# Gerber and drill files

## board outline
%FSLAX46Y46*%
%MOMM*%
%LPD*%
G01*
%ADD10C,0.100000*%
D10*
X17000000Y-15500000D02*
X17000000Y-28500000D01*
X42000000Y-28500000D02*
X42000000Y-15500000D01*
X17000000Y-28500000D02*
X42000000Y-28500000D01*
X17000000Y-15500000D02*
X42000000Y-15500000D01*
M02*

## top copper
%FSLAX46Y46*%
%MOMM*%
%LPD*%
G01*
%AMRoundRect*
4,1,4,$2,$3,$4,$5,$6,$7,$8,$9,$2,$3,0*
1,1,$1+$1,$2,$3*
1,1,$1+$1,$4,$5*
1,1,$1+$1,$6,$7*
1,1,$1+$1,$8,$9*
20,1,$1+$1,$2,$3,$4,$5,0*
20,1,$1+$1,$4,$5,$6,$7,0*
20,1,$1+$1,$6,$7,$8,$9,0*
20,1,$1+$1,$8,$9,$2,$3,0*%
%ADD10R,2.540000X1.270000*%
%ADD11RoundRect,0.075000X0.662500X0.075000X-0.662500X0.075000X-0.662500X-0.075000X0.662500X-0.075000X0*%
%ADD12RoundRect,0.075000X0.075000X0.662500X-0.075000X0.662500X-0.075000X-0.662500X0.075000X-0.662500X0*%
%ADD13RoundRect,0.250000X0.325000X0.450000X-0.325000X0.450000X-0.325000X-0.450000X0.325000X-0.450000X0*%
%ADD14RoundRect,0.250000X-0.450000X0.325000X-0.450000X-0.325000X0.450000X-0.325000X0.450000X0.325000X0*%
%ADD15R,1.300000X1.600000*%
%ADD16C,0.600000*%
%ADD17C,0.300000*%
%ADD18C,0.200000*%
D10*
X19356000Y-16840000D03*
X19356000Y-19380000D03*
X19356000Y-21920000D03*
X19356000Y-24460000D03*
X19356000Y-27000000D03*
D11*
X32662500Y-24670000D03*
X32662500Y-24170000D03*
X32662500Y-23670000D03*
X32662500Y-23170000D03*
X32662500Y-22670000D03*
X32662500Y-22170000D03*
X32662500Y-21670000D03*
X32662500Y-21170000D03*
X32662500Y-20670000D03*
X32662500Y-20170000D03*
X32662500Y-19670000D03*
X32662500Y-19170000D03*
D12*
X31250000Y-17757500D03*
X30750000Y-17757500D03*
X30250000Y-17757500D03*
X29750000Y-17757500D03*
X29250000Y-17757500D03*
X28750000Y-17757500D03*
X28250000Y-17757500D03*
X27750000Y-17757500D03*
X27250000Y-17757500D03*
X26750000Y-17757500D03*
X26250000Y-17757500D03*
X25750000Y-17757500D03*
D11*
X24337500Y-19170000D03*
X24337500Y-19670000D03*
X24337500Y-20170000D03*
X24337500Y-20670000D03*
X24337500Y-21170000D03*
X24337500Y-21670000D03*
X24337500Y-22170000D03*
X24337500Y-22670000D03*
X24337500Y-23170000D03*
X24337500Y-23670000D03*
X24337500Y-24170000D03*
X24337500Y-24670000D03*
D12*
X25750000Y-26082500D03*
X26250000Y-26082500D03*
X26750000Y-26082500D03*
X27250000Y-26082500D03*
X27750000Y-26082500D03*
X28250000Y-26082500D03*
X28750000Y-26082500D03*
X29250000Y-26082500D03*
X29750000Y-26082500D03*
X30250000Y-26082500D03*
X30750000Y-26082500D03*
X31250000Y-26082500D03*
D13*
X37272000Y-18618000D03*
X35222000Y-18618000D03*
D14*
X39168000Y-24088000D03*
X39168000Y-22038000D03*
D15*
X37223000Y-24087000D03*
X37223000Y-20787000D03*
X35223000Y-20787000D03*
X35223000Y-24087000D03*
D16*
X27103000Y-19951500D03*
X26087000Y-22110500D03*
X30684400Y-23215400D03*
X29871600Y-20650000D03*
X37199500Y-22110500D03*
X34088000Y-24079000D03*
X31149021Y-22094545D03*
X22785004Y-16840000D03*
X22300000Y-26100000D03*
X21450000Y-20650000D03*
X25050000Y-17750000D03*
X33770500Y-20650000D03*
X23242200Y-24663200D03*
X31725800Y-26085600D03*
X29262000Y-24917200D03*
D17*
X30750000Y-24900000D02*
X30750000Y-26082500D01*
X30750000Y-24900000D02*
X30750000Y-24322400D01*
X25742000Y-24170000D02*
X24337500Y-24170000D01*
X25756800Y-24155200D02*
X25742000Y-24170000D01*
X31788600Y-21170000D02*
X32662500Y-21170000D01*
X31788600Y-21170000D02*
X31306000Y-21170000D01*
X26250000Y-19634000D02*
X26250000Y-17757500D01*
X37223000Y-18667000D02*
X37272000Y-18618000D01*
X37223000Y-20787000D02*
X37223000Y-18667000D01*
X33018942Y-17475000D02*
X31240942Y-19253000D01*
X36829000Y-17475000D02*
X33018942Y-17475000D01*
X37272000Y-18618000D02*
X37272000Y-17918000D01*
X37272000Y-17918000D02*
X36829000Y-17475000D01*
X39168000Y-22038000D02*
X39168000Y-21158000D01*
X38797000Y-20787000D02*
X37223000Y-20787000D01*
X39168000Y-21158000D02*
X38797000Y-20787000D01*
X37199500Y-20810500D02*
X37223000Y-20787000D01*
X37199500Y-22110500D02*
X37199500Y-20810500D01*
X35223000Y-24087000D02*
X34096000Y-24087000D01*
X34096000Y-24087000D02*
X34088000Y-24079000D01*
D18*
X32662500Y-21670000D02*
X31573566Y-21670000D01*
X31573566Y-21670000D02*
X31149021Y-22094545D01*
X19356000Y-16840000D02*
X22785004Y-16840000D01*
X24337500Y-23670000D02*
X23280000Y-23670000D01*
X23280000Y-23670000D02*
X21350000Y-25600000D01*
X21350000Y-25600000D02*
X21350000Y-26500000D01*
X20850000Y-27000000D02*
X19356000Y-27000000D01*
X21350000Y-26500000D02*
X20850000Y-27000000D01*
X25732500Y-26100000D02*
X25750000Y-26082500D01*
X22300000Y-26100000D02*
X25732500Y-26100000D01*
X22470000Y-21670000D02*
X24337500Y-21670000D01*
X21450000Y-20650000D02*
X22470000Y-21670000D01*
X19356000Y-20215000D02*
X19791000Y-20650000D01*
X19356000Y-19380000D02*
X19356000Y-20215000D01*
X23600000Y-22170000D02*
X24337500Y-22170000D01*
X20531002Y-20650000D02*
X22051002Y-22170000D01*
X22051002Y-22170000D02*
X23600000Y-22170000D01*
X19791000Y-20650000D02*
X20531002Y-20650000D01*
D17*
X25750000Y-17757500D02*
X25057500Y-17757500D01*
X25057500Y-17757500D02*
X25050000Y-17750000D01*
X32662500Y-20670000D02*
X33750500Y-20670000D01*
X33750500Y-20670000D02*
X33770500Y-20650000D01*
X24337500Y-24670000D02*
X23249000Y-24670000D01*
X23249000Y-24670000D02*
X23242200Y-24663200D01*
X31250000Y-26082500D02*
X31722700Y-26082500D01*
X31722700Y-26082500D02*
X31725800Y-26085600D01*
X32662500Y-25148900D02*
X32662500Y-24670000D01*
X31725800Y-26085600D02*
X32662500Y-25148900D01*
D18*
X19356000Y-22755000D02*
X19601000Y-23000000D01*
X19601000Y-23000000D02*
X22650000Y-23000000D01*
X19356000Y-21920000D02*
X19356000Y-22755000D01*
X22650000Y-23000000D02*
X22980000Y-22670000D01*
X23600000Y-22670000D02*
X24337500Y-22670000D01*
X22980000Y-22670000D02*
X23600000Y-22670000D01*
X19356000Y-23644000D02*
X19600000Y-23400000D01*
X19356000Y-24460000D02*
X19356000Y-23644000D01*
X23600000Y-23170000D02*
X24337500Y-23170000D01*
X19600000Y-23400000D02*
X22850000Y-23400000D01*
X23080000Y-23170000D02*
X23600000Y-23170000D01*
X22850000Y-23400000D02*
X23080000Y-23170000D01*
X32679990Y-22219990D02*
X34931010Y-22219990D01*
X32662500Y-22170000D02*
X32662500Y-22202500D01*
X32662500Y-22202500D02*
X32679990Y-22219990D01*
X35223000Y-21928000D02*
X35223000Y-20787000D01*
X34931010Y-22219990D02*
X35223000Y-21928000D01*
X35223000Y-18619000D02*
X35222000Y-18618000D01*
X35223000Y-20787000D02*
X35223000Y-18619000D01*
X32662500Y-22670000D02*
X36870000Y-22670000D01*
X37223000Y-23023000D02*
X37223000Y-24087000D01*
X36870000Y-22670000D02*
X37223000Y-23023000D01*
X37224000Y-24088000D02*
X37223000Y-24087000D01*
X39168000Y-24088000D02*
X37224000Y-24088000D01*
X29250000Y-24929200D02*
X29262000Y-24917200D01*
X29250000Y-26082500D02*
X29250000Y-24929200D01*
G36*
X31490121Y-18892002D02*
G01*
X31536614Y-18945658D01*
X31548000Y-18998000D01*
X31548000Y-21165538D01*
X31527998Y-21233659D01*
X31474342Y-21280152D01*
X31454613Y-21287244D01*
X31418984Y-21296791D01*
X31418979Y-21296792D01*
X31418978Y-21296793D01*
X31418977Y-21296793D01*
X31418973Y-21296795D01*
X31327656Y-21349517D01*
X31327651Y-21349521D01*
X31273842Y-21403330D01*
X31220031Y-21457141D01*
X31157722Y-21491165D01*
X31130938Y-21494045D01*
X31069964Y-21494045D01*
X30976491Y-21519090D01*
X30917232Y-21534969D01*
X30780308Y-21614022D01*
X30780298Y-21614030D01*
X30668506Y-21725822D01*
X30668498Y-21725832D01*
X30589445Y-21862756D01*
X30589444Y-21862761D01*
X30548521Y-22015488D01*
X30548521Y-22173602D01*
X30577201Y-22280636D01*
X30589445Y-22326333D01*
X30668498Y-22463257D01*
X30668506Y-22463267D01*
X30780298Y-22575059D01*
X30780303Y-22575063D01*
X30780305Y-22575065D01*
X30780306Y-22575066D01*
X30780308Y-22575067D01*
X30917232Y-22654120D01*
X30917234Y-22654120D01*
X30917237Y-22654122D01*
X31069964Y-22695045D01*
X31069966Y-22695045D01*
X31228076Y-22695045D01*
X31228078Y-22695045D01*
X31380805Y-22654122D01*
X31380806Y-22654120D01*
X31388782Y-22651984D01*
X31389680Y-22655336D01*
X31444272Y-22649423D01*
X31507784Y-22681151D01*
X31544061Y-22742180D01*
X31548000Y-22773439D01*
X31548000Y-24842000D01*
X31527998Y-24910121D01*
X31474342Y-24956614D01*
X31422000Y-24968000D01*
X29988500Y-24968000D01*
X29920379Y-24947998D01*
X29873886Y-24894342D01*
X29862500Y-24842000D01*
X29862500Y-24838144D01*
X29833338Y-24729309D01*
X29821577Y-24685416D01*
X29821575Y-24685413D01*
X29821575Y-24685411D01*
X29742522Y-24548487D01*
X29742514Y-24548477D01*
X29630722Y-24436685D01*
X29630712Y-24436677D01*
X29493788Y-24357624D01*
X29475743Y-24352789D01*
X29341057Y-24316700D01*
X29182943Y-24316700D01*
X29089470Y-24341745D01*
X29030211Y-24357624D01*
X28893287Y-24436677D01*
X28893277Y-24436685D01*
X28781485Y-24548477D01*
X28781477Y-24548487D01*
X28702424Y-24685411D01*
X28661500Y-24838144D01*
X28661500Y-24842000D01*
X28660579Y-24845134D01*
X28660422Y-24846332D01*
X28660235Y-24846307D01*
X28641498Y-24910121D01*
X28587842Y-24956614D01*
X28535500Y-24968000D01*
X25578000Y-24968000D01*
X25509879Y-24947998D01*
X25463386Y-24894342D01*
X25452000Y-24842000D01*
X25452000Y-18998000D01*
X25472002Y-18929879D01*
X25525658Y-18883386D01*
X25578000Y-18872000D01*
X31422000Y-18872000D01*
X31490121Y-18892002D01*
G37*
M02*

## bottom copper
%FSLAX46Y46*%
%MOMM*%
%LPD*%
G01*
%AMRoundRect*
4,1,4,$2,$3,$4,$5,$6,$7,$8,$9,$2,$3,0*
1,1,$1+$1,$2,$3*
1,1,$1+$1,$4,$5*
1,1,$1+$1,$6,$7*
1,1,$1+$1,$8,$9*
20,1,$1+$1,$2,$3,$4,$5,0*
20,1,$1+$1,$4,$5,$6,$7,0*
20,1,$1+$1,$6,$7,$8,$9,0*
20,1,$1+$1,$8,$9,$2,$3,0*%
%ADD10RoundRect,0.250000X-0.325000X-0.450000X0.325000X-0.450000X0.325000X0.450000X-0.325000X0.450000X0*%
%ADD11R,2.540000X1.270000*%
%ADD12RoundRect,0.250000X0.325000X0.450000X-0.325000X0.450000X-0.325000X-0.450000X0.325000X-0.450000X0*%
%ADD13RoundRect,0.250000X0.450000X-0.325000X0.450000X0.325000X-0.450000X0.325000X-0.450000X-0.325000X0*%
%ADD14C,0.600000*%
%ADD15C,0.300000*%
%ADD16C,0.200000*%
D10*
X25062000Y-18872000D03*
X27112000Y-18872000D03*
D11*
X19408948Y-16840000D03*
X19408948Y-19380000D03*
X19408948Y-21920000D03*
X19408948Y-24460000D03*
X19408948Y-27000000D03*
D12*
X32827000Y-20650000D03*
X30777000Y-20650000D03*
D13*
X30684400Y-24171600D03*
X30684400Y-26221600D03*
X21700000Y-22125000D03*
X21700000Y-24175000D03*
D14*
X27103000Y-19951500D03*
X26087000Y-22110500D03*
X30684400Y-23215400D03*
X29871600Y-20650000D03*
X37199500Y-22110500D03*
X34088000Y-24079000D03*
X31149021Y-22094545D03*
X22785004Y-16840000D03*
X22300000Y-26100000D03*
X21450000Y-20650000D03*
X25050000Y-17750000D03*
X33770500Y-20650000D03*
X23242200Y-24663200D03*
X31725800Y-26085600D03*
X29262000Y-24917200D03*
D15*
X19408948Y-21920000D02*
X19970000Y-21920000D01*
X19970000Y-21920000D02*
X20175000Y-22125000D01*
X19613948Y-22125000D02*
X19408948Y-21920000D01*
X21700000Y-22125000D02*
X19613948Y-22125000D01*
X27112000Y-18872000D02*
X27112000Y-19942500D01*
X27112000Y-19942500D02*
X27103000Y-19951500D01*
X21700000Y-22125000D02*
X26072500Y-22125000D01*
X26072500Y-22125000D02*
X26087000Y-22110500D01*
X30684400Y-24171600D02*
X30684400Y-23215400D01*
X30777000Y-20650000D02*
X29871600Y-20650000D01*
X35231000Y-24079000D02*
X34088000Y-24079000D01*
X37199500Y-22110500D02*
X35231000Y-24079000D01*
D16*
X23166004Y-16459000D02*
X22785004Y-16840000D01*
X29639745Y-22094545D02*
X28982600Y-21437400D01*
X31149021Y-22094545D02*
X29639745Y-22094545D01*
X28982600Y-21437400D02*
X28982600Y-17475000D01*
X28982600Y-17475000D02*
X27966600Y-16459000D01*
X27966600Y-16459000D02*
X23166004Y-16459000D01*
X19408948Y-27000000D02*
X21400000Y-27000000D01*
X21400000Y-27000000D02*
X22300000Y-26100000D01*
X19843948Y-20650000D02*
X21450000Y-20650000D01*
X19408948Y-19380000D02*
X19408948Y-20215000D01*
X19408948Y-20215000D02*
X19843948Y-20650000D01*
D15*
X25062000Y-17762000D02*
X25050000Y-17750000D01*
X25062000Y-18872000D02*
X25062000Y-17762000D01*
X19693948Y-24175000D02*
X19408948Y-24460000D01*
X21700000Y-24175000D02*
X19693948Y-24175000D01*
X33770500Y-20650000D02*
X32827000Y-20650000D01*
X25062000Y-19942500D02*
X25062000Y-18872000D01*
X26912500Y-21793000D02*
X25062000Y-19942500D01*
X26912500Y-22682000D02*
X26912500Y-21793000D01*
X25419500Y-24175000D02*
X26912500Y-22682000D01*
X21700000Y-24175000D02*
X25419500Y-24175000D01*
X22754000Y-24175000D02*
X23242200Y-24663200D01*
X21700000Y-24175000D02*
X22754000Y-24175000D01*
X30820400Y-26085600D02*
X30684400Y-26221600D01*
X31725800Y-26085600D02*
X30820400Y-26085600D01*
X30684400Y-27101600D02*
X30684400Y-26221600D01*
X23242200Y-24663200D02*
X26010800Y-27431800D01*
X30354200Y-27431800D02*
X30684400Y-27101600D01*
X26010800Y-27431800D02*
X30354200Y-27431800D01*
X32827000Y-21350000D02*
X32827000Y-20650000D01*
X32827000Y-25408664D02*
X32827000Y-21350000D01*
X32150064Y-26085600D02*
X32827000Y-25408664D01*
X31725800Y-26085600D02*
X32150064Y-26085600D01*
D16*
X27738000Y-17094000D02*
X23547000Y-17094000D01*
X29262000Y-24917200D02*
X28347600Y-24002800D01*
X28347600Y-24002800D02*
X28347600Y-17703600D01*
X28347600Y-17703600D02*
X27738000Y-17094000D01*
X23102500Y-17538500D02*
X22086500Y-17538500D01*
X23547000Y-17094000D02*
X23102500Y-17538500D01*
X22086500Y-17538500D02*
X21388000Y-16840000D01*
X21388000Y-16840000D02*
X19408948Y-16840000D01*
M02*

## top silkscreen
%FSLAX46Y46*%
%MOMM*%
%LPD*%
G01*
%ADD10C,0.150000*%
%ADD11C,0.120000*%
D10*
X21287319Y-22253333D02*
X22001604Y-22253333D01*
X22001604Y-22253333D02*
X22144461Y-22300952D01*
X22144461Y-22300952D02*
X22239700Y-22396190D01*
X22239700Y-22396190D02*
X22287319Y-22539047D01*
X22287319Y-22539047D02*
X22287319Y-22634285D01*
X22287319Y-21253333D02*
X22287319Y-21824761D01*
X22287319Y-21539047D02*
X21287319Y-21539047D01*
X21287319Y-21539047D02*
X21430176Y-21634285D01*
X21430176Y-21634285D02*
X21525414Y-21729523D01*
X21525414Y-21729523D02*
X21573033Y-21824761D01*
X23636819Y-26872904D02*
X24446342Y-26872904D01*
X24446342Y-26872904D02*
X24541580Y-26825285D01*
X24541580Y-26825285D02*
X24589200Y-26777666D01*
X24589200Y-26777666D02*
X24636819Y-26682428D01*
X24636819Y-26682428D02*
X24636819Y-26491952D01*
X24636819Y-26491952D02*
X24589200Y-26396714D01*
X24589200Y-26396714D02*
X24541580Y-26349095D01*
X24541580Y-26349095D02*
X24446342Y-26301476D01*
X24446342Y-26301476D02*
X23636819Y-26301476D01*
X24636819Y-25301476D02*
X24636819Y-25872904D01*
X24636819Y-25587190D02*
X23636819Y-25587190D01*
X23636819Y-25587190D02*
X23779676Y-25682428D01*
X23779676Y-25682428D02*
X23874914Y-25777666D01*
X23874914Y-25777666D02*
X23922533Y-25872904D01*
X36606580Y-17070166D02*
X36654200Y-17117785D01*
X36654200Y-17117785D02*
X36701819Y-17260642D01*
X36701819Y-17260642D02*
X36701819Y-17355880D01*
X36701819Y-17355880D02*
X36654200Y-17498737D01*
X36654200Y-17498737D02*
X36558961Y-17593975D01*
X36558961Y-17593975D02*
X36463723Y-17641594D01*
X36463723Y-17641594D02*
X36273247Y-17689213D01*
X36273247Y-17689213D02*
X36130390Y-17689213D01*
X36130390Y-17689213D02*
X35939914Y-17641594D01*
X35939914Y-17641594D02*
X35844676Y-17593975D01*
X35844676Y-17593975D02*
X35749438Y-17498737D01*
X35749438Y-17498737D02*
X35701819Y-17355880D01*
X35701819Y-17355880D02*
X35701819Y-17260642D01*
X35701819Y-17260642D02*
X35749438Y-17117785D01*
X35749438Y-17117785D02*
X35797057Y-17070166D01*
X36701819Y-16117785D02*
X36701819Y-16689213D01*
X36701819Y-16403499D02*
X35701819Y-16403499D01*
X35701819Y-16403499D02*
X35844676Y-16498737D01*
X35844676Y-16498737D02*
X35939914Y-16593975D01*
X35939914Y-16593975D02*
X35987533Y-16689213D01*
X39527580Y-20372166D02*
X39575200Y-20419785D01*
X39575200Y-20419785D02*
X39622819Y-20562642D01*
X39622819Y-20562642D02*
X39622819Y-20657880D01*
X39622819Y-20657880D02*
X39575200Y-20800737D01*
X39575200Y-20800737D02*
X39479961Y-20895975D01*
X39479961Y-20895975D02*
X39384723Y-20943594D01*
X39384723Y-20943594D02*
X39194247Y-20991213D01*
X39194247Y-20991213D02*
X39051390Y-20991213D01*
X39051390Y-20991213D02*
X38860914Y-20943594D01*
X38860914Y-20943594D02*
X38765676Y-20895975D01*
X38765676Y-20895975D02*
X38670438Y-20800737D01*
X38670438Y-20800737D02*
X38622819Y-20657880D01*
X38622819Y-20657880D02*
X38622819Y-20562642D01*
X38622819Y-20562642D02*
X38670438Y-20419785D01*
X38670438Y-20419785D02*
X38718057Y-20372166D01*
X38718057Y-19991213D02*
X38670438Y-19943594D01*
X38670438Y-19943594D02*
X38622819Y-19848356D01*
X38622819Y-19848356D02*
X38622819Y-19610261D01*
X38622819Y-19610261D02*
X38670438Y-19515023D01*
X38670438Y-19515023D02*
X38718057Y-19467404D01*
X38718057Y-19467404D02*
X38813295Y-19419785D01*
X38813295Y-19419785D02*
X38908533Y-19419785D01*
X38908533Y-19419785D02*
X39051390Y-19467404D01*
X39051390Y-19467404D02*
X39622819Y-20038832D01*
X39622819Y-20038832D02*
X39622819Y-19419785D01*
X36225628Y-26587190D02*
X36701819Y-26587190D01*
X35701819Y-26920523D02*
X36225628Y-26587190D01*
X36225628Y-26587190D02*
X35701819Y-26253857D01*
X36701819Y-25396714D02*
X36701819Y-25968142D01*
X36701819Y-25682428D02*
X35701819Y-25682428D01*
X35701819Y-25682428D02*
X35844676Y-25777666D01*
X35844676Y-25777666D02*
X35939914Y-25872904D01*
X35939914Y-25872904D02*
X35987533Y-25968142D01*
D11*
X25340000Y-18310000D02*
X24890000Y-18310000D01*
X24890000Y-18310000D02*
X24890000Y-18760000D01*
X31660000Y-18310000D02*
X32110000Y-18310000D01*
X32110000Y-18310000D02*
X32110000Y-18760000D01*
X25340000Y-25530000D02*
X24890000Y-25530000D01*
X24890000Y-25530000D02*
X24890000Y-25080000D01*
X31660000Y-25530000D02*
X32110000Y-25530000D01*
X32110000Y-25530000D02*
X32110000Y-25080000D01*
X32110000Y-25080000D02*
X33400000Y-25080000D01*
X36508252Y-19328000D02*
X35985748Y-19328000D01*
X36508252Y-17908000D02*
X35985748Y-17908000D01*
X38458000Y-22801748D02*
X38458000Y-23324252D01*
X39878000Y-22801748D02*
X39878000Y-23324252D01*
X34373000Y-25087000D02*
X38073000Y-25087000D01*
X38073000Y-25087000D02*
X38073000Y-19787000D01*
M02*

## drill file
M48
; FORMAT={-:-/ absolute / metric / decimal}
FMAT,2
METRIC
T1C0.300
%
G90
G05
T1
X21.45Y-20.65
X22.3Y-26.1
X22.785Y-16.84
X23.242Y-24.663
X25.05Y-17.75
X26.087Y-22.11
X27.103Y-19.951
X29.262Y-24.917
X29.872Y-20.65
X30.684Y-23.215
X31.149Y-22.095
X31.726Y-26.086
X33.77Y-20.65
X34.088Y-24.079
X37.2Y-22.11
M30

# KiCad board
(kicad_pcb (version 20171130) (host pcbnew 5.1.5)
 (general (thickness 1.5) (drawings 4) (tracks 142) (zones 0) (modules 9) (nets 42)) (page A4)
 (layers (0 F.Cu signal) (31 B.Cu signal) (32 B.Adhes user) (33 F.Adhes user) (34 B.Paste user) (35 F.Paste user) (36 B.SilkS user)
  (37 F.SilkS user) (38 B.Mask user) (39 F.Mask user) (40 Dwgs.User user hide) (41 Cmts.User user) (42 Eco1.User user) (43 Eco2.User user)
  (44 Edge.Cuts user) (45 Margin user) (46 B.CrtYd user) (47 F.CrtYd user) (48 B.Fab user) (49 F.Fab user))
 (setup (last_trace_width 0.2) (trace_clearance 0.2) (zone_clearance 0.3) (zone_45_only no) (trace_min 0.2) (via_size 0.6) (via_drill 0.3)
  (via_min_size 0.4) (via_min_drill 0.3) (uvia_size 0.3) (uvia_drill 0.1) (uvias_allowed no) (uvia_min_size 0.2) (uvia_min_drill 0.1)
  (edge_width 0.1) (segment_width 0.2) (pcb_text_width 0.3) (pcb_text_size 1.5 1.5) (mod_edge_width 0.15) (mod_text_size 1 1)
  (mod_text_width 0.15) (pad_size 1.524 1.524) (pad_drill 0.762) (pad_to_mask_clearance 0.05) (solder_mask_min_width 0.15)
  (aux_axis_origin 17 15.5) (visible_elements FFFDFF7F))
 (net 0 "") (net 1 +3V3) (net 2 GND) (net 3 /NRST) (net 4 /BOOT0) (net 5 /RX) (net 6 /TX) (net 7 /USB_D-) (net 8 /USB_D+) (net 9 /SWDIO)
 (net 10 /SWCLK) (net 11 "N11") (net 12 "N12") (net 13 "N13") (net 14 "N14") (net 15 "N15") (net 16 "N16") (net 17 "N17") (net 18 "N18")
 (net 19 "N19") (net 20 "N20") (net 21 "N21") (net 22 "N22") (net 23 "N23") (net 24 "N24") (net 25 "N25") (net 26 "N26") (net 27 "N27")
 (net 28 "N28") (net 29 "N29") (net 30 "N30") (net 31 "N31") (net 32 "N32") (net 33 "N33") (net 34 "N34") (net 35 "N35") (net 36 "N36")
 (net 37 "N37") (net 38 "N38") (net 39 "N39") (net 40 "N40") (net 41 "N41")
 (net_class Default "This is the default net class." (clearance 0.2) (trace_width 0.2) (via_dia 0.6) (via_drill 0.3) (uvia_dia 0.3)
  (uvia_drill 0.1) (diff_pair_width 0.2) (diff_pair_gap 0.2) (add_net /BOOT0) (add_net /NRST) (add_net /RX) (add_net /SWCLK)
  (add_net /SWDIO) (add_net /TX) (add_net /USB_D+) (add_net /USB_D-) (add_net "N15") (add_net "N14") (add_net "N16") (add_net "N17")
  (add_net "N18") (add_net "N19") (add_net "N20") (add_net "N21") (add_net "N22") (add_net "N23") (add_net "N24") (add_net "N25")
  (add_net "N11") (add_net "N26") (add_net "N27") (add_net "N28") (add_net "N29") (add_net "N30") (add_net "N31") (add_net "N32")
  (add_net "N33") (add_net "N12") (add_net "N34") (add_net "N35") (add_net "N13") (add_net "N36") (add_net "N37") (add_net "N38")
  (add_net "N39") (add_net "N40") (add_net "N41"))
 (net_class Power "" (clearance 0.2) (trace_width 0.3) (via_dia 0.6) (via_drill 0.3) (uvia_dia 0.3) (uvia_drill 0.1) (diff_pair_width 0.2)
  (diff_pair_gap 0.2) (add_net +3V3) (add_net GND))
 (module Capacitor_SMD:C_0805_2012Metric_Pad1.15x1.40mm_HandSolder (layer B.Cu) (at 26.087 18.872)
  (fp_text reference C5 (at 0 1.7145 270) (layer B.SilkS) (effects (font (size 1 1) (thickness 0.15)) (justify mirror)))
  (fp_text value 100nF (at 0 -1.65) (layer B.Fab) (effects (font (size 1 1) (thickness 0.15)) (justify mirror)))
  (pad 1 smd roundrect (at -1.025 0) (size 1.15 1.4) (layers B.Cu B.Paste B.Mask) (roundrect_rratio 0.217391) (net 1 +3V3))
  (pad 2 smd roundrect (at 1.025 0) (size 1.15 1.4) (layers B.Cu B.Paste B.Mask) (roundrect_rratio 0.217391) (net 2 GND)))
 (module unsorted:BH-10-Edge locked (layer F.Cu) (at 19.356 21.92 270)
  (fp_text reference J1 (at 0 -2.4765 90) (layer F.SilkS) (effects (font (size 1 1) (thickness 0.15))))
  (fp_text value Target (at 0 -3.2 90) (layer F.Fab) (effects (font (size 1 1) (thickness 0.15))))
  (pad 1 smd rect (at -5.08 0 270) (size 1.27 2.54) (layers F.Cu F.Paste F.Mask) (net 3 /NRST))
  (pad 2 smd rect (at -5.08 -0.052948 270) (size 1.27 2.54) (layers B.Cu B.Paste B.Mask) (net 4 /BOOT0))
  (pad 3 smd rect (at -2.54 0 270) (size 1.27 2.54) (layers F.Cu F.Paste F.Mask) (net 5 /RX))
  (pad 4 smd rect (at -2.54 -0.052948 270) (size 1.27 2.54) (layers B.Cu B.Paste B.Mask) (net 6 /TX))
  (pad 5 smd rect (at 0 0 270) (size 1.27 2.54) (layers F.Cu F.Paste F.Mask) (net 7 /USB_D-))
  (pad 6 smd rect (at 0 -0.052948 270) (size 1.27 2.54) (layers B.Cu B.Paste B.Mask) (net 2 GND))
  (pad 7 smd rect (at 2.54 0 270) (size 1.27 2.54) (layers F.Cu F.Paste F.Mask) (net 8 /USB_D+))
  (pad 8 smd rect (at 2.54 -0.052948 270) (size 1.27 2.54) (layers B.Cu B.Paste B.Mask) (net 1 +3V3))
  (pad 9 smd rect (at 5.08 0 270) (size 1.27 2.54) (layers F.Cu F.Paste F.Mask) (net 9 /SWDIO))
  (pad 10 smd rect (at 5.08 -0.052948 270) (size 1.27 2.54) (layers B.Cu B.Paste B.Mask) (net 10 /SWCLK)))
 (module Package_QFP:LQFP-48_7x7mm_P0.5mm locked (layer F.Cu) (at 28.5 21.92 180)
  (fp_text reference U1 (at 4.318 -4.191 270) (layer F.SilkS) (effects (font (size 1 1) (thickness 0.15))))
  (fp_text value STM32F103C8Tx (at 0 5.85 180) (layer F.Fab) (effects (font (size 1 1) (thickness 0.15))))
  (fp_line (start 3.16 3.61) (end 3.61 3.61) (layer F.SilkS) (width 0.12))
  (fp_line (start 3.61 3.61) (end 3.61 3.16) (layer F.SilkS) (width 0.12))
  (fp_line (start -3.16 3.61) (end -3.61 3.61) (layer F.SilkS) (width 0.12))
  (fp_line (start -3.61 3.61) (end -3.61 3.16) (layer F.SilkS) (width 0.12))
  (fp_line (start 3.16 -3.61) (end 3.61 -3.61) (layer F.SilkS) (width 0.12))
  (fp_line (start 3.61 -3.61) (end 3.61 -3.16) (layer F.SilkS) (width 0.12))
  (fp_line (start -3.16 -3.61) (end -3.61 -3.61) (layer F.SilkS) (width 0.12))
  (fp_line (start -3.61 -3.61) (end -3.61 -3.16) (layer F.SilkS) (width 0.12))
  (fp_line (start -3.61 -3.16) (end -4.9 -3.16) (layer F.SilkS) (width 0.12))
  (pad 1 smd roundrect (at -4.1625 -2.75 180) (size 1.475 0.3) (layers F.Cu F.Paste F.Mask) (roundrect_rratio 0.25) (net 1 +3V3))
  (pad 2 smd roundrect (at -4.1625 -2.25 180) (size 1.475 0.3) (layers F.Cu F.Paste F.Mask) (roundrect_rratio 0.25) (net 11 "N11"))
  (pad 3 smd roundrect (at -4.1625 -1.75 180) (size 1.475 0.3) (layers F.Cu F.Paste F.Mask) (roundrect_rratio 0.25) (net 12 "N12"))
  (pad 4 smd roundrect (at -4.1625 -1.25 180) (size 1.475 0.3) (layers F.Cu F.Paste F.Mask) (roundrect_rratio 0.25) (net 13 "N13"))
  (pad 5 smd roundrect (at -4.1625 -0.75 180) (size 1.475 0.3) (layers F.Cu F.Paste F.Mask) (roundrect_rratio 0.25) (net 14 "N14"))
  (pad 6 smd roundrect (at -4.1625 -0.25 180) (size 1.475 0.3) (layers F.Cu F.Paste F.Mask) (roundrect_rratio 0.25) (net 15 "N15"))
  (pad 7 smd roundrect (at -4.1625 0.25 180) (size 1.475 0.3) (layers F.Cu F.Paste F.Mask) (roundrect_rratio 0.25) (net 3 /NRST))
  (pad 8 smd roundrect (at -4.1625 0.75 180) (size 1.475 0.3) (layers F.Cu F.Paste F.Mask) (roundrect_rratio 0.25) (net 2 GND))
  (pad 9 smd roundrect (at -4.1625 1.25 180) (size 1.475 0.3) (layers F.Cu F.Paste F.Mask) (roundrect_rratio 0.25) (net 1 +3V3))
  (pad 10 smd roundrect (at -4.1625 1.75 180) (size 1.475 0.3) (layers F.Cu F.Paste F.Mask) (roundrect_rratio 0.25) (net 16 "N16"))
  (pad 11 smd roundrect (at -4.1625 2.25 180) (size 1.475 0.3) (layers F.Cu F.Paste F.Mask) (roundrect_rratio 0.25) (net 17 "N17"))
  (pad 12 smd roundrect (at -4.1625 2.75 180) (size 1.475 0.3) (layers F.Cu F.Paste F.Mask) (roundrect_rratio 0.25) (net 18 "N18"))
  (pad 13 smd roundrect (at -2.75 4.1625 180) (size 0.3 1.475) (layers F.Cu F.Paste F.Mask) (roundrect_rratio 0.25) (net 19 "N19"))
  (pad 14 smd roundrect (at -2.25 4.1625 180) (size 0.3 1.475) (layers F.Cu F.Paste F.Mask) (roundrect_rratio 0.25) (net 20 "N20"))
  (pad 15 smd roundrect (at -1.75 4.1625 180) (size 0.3 1.475) (layers F.Cu F.Paste F.Mask) (roundrect_rratio 0.25) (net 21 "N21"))
  (pad 16 smd roundrect (at -1.25 4.1625 180) (size 0.3 1.475) (layers F.Cu F.Paste F.Mask) (roundrect_rratio 0.25) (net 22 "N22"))
  (pad 17 smd roundrect (at -0.75 4.1625 180) (size 0.3 1.475) (layers F.Cu F.Paste F.Mask) (roundrect_rratio 0.25) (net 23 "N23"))
  (pad 18 smd roundrect (at -0.25 4.1625 180) (size 0.3 1.475) (layers F.Cu F.Paste F.Mask) (roundrect_rratio 0.25) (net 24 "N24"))
  (pad 19 smd roundrect (at 0.25 4.1625 180) (size 0.3 1.475) (layers F.Cu F.Paste F.Mask) (roundrect_rratio 0.25) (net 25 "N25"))
  (pad 20 smd roundrect (at 0.75 4.1625 180) (size 0.3 1.475) (layers F.Cu F.Paste F.Mask) (roundrect_rratio 0.25) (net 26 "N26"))
  (pad 21 smd roundrect (at 1.25 4.1625 180) (size 0.3 1.475) (layers F.Cu F.Paste F.Mask) (roundrect_rratio 0.25) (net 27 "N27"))
  (pad 22 smd roundrect (at 1.75 4.1625 180) (size 0.3 1.475) (layers F.Cu F.Paste F.Mask) (roundrect_rratio 0.25) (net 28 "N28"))
  (pad 23 smd roundrect (at 2.25 4.1625 180) (size 0.3 1.475) (layers F.Cu F.Paste F.Mask) (roundrect_rratio 0.25) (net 2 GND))
  (pad 24 smd roundrect (at 2.75 4.1625 180) (size 0.3 1.475) (layers F.Cu F.Paste F.Mask) (roundrect_rratio 0.25) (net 1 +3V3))
  (pad 25 smd roundrect (at 4.1625 2.75 180) (size 1.475 0.3) (layers F.Cu F.Paste F.Mask) (roundrect_rratio 0.25) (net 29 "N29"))
  (pad 26 smd roundrect (at 4.1625 2.25 180) (size 1.475 0.3) (layers F.Cu F.Paste F.Mask) (roundrect_rratio 0.25) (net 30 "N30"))
  (pad 27 smd roundrect (at 4.1625 1.75 180) (size 1.475 0.3) (layers F.Cu F.Paste F.Mask) (roundrect_rratio 0.25) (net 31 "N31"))
  (pad 28 smd roundrect (at 4.1625 1.25 180) (size 1.475 0.3) (layers F.Cu F.Paste F.Mask) (roundrect_rratio 0.25) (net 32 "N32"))
  (pad 29 smd roundrect (at 4.1625 0.75 180) (size 1.475 0.3) (layers F.Cu F.Paste F.Mask) (roundrect_rratio 0.25) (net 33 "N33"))
  (pad 30 smd roundrect (at 4.1625 0.25 180) (size 1.475 0.3) (layers F.Cu F.Paste F.Mask) (roundrect_rratio 0.25) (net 6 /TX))
  (pad 31 smd roundrect (at 4.1625 -0.25 180) (size 1.475 0.3) (layers F.Cu F.Paste F.Mask) (roundrect_rratio 0.25) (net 5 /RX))
  (pad 32 smd roundrect (at 4.1625 -0.75 180) (size 1.475 0.3) (layers F.Cu F.Paste F.Mask) (roundrect_rratio 0.25) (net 7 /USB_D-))
  (pad 33 smd roundrect (at 4.1625 -1.25 180) (size 1.475 0.3) (layers F.Cu F.Paste F.Mask) (roundrect_rratio 0.25) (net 8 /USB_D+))
  (pad 34 smd roundrect (at 4.1625 -1.75 180) (size 1.475 0.3) (layers F.Cu F.Paste F.Mask) (roundrect_rratio 0.25) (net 9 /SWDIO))
  (pad 35 smd roundrect (at 4.1625 -2.25 180) (size 1.475 0.3) (layers F.Cu F.Paste F.Mask) (roundrect_rratio 0.25) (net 2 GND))
  (pad 36 smd roundrect (at 4.1625 -2.75 180) (size 1.475 0.3) (layers F.Cu F.Paste F.Mask) (roundrect_rratio 0.25) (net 1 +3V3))
  (pad 37 smd roundrect (at 2.75 -4.1625 180) (size 0.3 1.475) (layers F.Cu F.Paste F.Mask) (roundrect_rratio 0.25) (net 10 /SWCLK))
  (pad 38 smd roundrect (at 2.25 -4.1625 180) (size 0.3 1.475) (layers F.Cu F.Paste F.Mask) (roundrect_rratio 0.25) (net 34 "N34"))
  (pad 39 smd roundrect (at 1.75 -4.1625 180) (size 0.3 1.475) (layers F.Cu F.Paste F.Mask) (roundrect_rratio 0.25) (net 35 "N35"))
  (pad 40 smd roundrect (at 1.25 -4.1625 180) (size 0.3 1.475) (layers F.Cu F.Paste F.Mask) (roundrect_rratio 0.25) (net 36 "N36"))
  (pad 41 smd roundrect (at 0.75 -4.1625 180) (size 0.3 1.475) (layers F.Cu F.Paste F.Mask) (roundrect_rratio 0.25) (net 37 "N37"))
  (pad 42 smd roundrect (at 0.25 -4.1625 180) (size 0.3 1.475) (layers F.Cu F.Paste F.Mask) (roundrect_rratio 0.25) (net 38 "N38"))
  (pad 43 smd roundrect (at -0.25 -4.1625 180) (size 0.3 1.475) (layers F.Cu F.Paste F.Mask) (roundrect_rratio 0.25) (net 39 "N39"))
  (pad 44 smd roundrect (at -0.75 -4.1625 180) (size 0.3 1.475) (layers F.Cu F.Paste F.Mask) (roundrect_rratio 0.25) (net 4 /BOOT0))
  (pad 45 smd roundrect (at -1.25 -4.1625 180) (size 0.3 1.475) (layers F.Cu F.Paste F.Mask) (roundrect_rratio 0.25) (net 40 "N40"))
  (pad 46 smd roundrect (at -1.75 -4.1625 180) (size 0.3 1.475) (layers F.Cu F.Paste F.Mask) (roundrect_rratio 0.25) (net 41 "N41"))
  (pad 47 smd roundrect (at -2.25 -4.1625 180) (size 0.3 1.475) (layers F.Cu F.Paste F.Mask) (roundrect_rratio 0.25) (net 2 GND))
  (pad 48 smd roundrect (at -2.75 -4.1625 180) (size 0.3 1.475) (layers F.Cu F.Paste F.Mask) (roundrect_rratio 0.25) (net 1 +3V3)))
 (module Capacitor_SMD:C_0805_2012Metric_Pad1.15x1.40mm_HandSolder (layer F.Cu) (at 36.247 18.618 180)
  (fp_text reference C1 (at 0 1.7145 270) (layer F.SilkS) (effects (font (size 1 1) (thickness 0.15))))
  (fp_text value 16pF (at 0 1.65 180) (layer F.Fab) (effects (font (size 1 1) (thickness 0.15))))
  (fp_line (start -0.261252 -0.71) (end 0.261252 -0.71) (layer F.SilkS) (width 0.12))
  (fp_line (start -0.261252 0.71) (end 0.261252 0.71) (layer F.SilkS) (width 0.12))
  (pad 1 smd roundrect (at -1.025 0 180) (size 1.15 1.4) (layers F.Cu F.Paste F.Mask) (roundrect_rratio 0.217391) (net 2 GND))
  (pad 2 smd roundrect (at 1.025 0 180) (size 1.15 1.4) (layers F.Cu F.Paste F.Mask) (roundrect_rratio 0.217391) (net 15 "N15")))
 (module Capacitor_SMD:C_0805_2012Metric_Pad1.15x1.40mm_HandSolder (layer F.Cu) (at 39.168 23.063 270)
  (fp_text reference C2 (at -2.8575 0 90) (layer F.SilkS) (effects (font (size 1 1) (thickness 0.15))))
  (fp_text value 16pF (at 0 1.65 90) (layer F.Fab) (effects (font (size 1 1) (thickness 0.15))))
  (fp_line (start -0.261252 0.71) (end 0.261252 0.71) (layer F.SilkS) (width 0.12))
  (fp_line (start -0.261252 -0.71) (end 0.261252 -0.71) (layer F.SilkS) (width 0.12))
  (pad 2 smd roundrect (at 1.025 0 270) (size 1.15 1.4) (layers F.Cu F.Paste F.Mask) (roundrect_rratio 0.217391) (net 14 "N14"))
  (pad 1 smd roundrect (at -1.025 0 270) (size 1.15 1.4) (layers F.Cu F.Paste F.Mask) (roundrect_rratio 0.217391) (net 2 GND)))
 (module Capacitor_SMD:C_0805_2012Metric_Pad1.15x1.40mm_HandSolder (layer B.Cu) (at 31.802 20.65 180)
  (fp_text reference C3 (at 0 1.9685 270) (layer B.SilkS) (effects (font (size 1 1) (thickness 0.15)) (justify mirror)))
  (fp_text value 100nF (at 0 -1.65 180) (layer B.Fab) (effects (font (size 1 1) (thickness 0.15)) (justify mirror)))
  (pad 1 smd roundrect (at -1.025 0 180) (size 1.15 1.4) (layers B.Cu B.Paste B.Mask) (roundrect_rratio 0.217391) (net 1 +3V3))
  (pad 2 smd roundrect (at 1.025 0 180) (size 1.15 1.4) (layers B.Cu B.Paste B.Mask) (roundrect_rratio 0.217391) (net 2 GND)))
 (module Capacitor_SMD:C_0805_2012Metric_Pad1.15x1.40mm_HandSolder (layer B.Cu) (at 30.6844 25.1966 90)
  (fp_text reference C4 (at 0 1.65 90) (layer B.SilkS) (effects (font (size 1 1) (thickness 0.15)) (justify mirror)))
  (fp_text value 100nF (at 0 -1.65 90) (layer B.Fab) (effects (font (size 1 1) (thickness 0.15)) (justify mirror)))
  (pad 2 smd roundrect (at 1.025 0 90) (size 1.15 1.4) (layers B.Cu B.Paste B.Mask) (roundrect_rratio 0.217391) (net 2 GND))
  (pad 1 smd roundrect (at -1.025 0 90) (size 1.15 1.4) (layers B.Cu B.Paste B.Mask) (roundrect_rratio 0.217391) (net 1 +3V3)))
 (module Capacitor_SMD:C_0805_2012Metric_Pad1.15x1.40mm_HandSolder (layer B.Cu) (at 21.7 23.15 90)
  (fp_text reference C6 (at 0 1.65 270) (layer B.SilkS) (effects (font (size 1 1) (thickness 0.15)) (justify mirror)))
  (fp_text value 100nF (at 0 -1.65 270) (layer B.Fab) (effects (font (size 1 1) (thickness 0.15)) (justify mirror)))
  (pad 2 smd roundrect (at 1.025 0 90) (size 1.15 1.4) (layers B.Cu B.Paste B.Mask) (roundrect_rratio 0.217391) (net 2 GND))
  (pad 1 smd roundrect (at -1.025 0 90) (size 1.15 1.4) (layers B.Cu B.Paste B.Mask) (roundrect_rratio 0.217391) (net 1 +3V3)))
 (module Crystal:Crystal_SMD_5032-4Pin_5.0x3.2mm (layer F.Cu) (at 36.223 22.437 90)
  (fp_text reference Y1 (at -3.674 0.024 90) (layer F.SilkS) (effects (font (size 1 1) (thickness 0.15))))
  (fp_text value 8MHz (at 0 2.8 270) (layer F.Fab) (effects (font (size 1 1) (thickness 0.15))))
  (fp_line (start -2.65 -1.85) (end -2.65 1.85) (layer F.SilkS) (width 0.12))
  (fp_line (start -2.65 1.85) (end 2.65 1.85) (layer F.SilkS) (width 0.12))
  (pad 1 smd rect (at -1.65 1 90) (size 1.6 1.3) (layers F.Cu F.Paste F.Mask) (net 14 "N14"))
  (pad 2 smd rect (at 1.65 1 90) (size 1.6 1.3) (layers F.Cu F.Paste F.Mask) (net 2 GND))
  (pad 3 smd rect (at 1.65 -1 90) (size 1.6 1.3) (layers F.Cu F.Paste F.Mask) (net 15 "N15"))
  (pad 4 smd rect (at -1.65 -1 90) (size 1.6 1.3) (layers F.Cu F.Paste F.Mask) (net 2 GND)))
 (gr_line (start 17 15.5) (end 17 28.5) (layer Edge.Cuts) (width 0.1))
 (gr_line (start 42 28.5) (end 42 15.5) (layer Edge.Cuts) (width 0.1))
 (gr_line (start 17 28.5) (end 42 28.5) (layer Edge.Cuts) (width 0.1))
 (gr_line (start 17 15.5) (end 42 15.5) (layer Edge.Cuts) (width 0.1))
 (segment (start 30.75 24.9) (end 30.75 26.0825) (width 0.3) (layer F.Cu) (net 2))
 (segment (start 19.408948 21.92) (end 19.97 21.92) (width 0.3) (layer B.Cu) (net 2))
 (segment (start 19.97 21.92) (end 20.175 22.125) (width 0.3) (layer B.Cu) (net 2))
 (segment (start 19.613948 22.125) (end 19.408948 21.92) (width 0.3) (layer B.Cu) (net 2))
 (segment (start 21.7 22.125) (end 19.613948 22.125) (width 0.3) (layer B.Cu) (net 2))
 (segment (start 27.112 18.872) (end 27.112 19.9425) (width 0.3) (layer B.Cu) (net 2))
 (via (at 27.103 19.9515) (size 0.6) (drill 0.3) (layers F.Cu B.Cu) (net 2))
 (segment (start 27.112 19.9425) (end 27.103 19.9515) (width 0.3) (layer B.Cu) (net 2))
 (via (at 26.087 22.1105) (size 0.6) (drill 0.3) (layers F.Cu B.Cu) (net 2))
 (segment (start 21.7 22.125) (end 26.0725 22.125) (width 0.3) (layer B.Cu) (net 2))
 (segment (start 26.0725 22.125) (end 26.087 22.1105) (width 0.3) (layer B.Cu) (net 2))
 (via (at 30.6844 23.2154) (size 0.6) (drill 0.3) (layers F.Cu B.Cu) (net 2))
 (segment (start 30.6844 24.1716) (end 30.6844 23.2154) (width 0.3) (layer B.Cu) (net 2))
 (segment (start 30.777 20.65) (end 29.8716 20.65) (width 0.3) (layer B.Cu) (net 2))
 (via (at 29.8716 20.65) (size 0.6) (drill 0.3) (layers F.Cu B.Cu) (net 2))
 (segment (start 30.75 24.9) (end 30.75 24.3224) (width 0.3) (layer F.Cu) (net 2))
 (segment (start 25.742 24.17) (end 24.3375 24.17) (width 0.3) (layer F.Cu) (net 2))
 (segment (start 25.7568 24.1552) (end 25.742 24.17) (width 0.3) (layer F.Cu) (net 2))
 (segment (start 31.7886 21.17) (end 32.6625 21.17) (width 0.3) (layer F.Cu) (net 2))
 (segment (start 31.7886 21.17) (end 31.306 21.17) (width 0.3) (layer F.Cu) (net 2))
 (segment (start 26.25 19.634) (end 26.25 17.7575) (width 0.3) (layer F.Cu) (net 2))
 (segment (start 37.223 18.667) (end 37.272 18.618) (width 0.3) (layer F.Cu) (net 2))
 (segment (start 37.223 20.787) (end 37.223 18.667) (width 0.3) (layer F.Cu) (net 2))
 (segment (start 33.018942 17.475) (end 31.240942 19.253) (width 0.3) (layer F.Cu) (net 2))
 (segment (start 36.829 17.475) (end 33.018942 17.475) (width 0.3) (layer F.Cu) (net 2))
 (segment (start 37.272 18.618) (end 37.272 17.918) (width 0.3) (layer F.Cu) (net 2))
 (segment (start 37.272 17.918) (end 36.829 17.475) (width 0.3) (layer F.Cu) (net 2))
 (segment (start 39.168 22.038) (end 39.168 21.158) (width 0.3) (layer F.Cu) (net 2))
 (segment (start 38.797 20.787) (end 37.223 20.787) (width 0.3) (layer F.Cu) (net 2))
 (segment (start 39.168 21.158) (end 38.797 20.787) (width 0.3) (layer F.Cu) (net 2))
 (via (at 37.1995 22.1105) (size 0.6) (drill 0.3) (layers F.Cu B.Cu) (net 2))
 (segment (start 37.1995 20.8105) (end 37.223 20.787) (width 0.3) (layer F.Cu) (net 2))
 (segment (start 37.1995 22.1105) (end 37.1995 20.8105) (width 0.3) (layer F.Cu) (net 2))
 (segment (start 35.231 24.079) (end 34.088 24.079) (width 0.3) (layer B.Cu) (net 2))
 (segment (start 37.1995 22.1105) (end 35.231 24.079) (width 0.3) (layer B.Cu) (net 2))
 (segment (start 35.223 24.087) (end 34.096 24.087) (width 0.3) (layer F.Cu) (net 2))
 (via (at 34.088 24.079) (size 0.6) (drill 0.3) (layers F.Cu B.Cu) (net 2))
 (segment (start 34.096 24.087) (end 34.088 24.079) (width 0.3) (layer F.Cu) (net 2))
 (via (at 31.149021 22.094545) (size 0.6) (drill 0.3) (layers F.Cu B.Cu) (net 3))
 (segment (start 32.6625 21.67) (end 31.573566 21.67) (width 0.2) (layer F.Cu) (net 3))
 (segment (start 31.573566 21.67) (end 31.149021 22.094545) (width 0.2) (layer F.Cu) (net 3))
 (via (at 22.785004 16.84) (size 0.6) (drill 0.3) (layers F.Cu B.Cu) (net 3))
 (segment (start 19.356 16.84) (end 22.785004 16.84) (width 0.2) (layer F.Cu) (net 3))
 (segment (start 23.166004 16.459) (end 22.785004 16.84) (width 0.2) (layer B.Cu) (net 3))
 (segment (start 29.639745 22.094545) (end 28.9826 21.4374) (width 0.2) (layer B.Cu) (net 3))
 (segment (start 31.149021 22.094545) (end 29.639745 22.094545) (width 0.2) (layer B.Cu) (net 3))
 (segment (start 28.9826 21.4374) (end 28.9826 17.475) (width 0.2) (layer B.Cu) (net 3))
 (segment (start 28.9826 17.475) (end 27.9666 16.459) (width 0.2) (layer B.Cu) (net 3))
 (segment (start 27.9666 16.459) (end 23.166004 16.459) (width 0.2) (layer B.Cu) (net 3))
 (segment (start 24.3375 23.67) (end 23.28 23.67) (width 0.2) (layer F.Cu) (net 9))
 (segment (start 23.28 23.67) (end 21.35 25.6) (width 0.2) (layer F.Cu) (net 9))
 (segment (start 21.35 25.6) (end 21.35 26.5) (width 0.2) (layer F.Cu) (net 9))
 (segment (start 20.85 27) (end 19.356 27) (width 0.2) (layer F.Cu) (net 9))
 (segment (start 21.35 26.5) (end 20.85 27) (width 0.2) (layer F.Cu) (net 9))
 (via (at 22.3 26.1) (size 0.6) (drill 0.3) (layers F.Cu B.Cu) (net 10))
 (segment (start 19.408948 27) (end 21.4 27) (width 0.2) (layer B.Cu) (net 10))
 (segment (start 21.4 27) (end 22.3 26.1) (width 0.2) (layer B.Cu) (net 10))
 (segment (start 25.7325 26.1) (end 25.75 26.0825) (width 0.2) (layer F.Cu) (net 10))
 (segment (start 22.3 26.1) (end 25.7325 26.1) (width 0.2) (layer F.Cu) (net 10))
 (via (at 21.45 20.65) (size 0.6) (drill 0.3) (layers F.Cu B.Cu) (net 6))
 (segment (start 19.843948 20.65) (end 21.45 20.65) (width 0.2) (layer B.Cu) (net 6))
 (segment (start 19.408948 19.38) (end 19.408948 20.215) (width 0.2) (layer B.Cu) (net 6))
 (segment (start 19.408948 20.215) (end 19.843948 20.65) (width 0.2) (layer B.Cu) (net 6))
 (segment (start 22.47 21.67) (end 24.3375 21.67) (width 0.2) (layer F.Cu) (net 6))
 (segment (start 21.45 20.65) (end 22.47 21.67) (width 0.2) (layer F.Cu) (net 6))
 (segment (start 19.356 20.215) (end 19.791 20.65) (width 0.2) (layer F.Cu) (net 5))
 (segment (start 19.356 19.38) (end 19.356 20.215) (width 0.2) (layer F.Cu) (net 5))
 (segment (start 23.6 22.17) (end 24.3375 22.17) (width 0.2) (layer F.Cu) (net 5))
 (segment (start 20.531002 20.65) (end 22.051002 22.17) (width 0.2) (layer F.Cu) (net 5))
 (segment (start 22.051002 22.17) (end 23.6 22.17) (width 0.2) (layer F.Cu) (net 5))
 (segment (start 19.791 20.65) (end 20.531002 20.65) (width 0.2) (layer F.Cu) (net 5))
 (via (at 25.05 17.75) (size 0.6) (drill 0.3) (layers F.Cu B.Cu) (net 1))
 (segment (start 25.75 17.7575) (end 25.0575 17.7575) (width 0.3) (layer F.Cu) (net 1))
 (segment (start 25.0575 17.7575) (end 25.05 17.75) (width 0.3) (layer F.Cu) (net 1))
 (segment (start 25.062 17.762) (end 25.05 17.75) (width 0.3) (layer B.Cu) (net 1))
 (segment (start 25.062 18.872) (end 25.062 17.762) (width 0.3) (layer B.Cu) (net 1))
 (segment (start 19.693948 24.175) (end 19.408948 24.46) (width 0.3) (layer B.Cu) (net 1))
 (segment (start 21.7 24.175) (end 19.693948 24.175) (width 0.3) (layer B.Cu) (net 1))
 (via (at 33.7705 20.65) (size 0.6) (drill 0.3) (layers F.Cu B.Cu) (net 1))
 (segment (start 32.6625 20.67) (end 33.7505 20.67) (width 0.3) (layer F.Cu) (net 1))
 (segment (start 33.7505 20.67) (end 33.7705 20.65) (width 0.3) (layer F.Cu) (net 1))
 (segment (start 33.7705 20.65) (end 32.827 20.65) (width 0.3) (layer B.Cu) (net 1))
 (segment (start 25.062 19.9425) (end 25.062 18.872) (width 0.3) (layer B.Cu) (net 1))
 (segment (start 26.9125 21.793) (end 25.062 19.9425) (width 0.3) (layer B.Cu) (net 1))
 (segment (start 26.9125 22.682) (end 26.9125 21.793) (width 0.3) (layer B.Cu) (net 1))
 (segment (start 25.4195 24.175) (end 26.9125 22.682) (width 0.3) (layer B.Cu) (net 1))
 (segment (start 21.7 24.175) (end 25.4195 24.175) (width 0.3) (layer B.Cu) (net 1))
 (via (at 23.2422 24.6632) (size 0.6) (drill 0.3) (layers F.Cu B.Cu) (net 1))
 (segment (start 24.3375 24.67) (end 23.249 24.67) (width 0.3) (layer F.Cu) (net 1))
 (segment (start 23.249 24.67) (end 23.2422 24.6632) (width 0.3) (layer F.Cu) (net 1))
 (segment (start 22.754 24.175) (end 23.2422 24.6632) (width 0.3) (layer B.Cu) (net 1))
 (segment (start 21.7 24.175) (end 22.754 24.175) (width 0.3) (layer B.Cu) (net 1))
 (via (at 31.7258 26.0856) (size 0.6) (drill 0.3) (layers F.Cu B.Cu) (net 1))
 (segment (start 31.25 26.0825) (end 31.7227 26.0825) (width 0.3) (layer F.Cu) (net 1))
 (segment (start 31.7227 26.0825) (end 31.7258 26.0856) (width 0.3) (layer F.Cu) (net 1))
 (segment (start 30.8204 26.0856) (end 30.6844 26.2216) (width 0.3) (layer B.Cu) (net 1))
 (segment (start 31.7258 26.0856) (end 30.8204 26.0856) (width 0.3) (layer B.Cu) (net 1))
 (segment (start 30.6844 27.1016) (end 30.6844 26.2216) (width 0.3) (layer B.Cu) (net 1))
 (segment (start 23.2422 24.6632) (end 26.0108 27.4318) (width 0.3) (layer B.Cu) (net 1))
 (segment (start 30.3542 27.4318) (end 30.6844 27.1016) (width 0.3) (layer B.Cu) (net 1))
 (segment (start 26.0108 27.4318) (end 30.3542 27.4318) (width 0.3) (layer B.Cu) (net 1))
 (segment (start 32.827 21.35) (end 32.827 20.65) (width 0.3) (layer B.Cu) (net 1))
 (segment (start 32.827 25.408664) (end 32.827 21.35) (width 0.3) (layer B.Cu) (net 1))
 (segment (start 32.150064 26.0856) (end 32.827 25.408664) (width 0.3) (layer B.Cu) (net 1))
 (segment (start 31.7258 26.0856) (end 32.150064 26.0856) (width 0.3) (layer B.Cu) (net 1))
 (segment (start 32.6625 25.1489) (end 32.6625 24.67) (width 0.3) (layer F.Cu) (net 1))
 (segment (start 31.7258 26.0856) (end 32.6625 25.1489) (width 0.3) (layer F.Cu) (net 1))
 (segment (start 19.356 22.755) (end 19.601 23) (width 0.2) (layer F.Cu) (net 7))
 (segment (start 19.601 23) (end 22.65 23) (width 0.2) (layer F.Cu) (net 7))
 (segment (start 19.356 21.92) (end 19.356 22.755) (width 0.2) (layer F.Cu) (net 7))
 (segment (start 22.65 23) (end 22.98 22.67) (width 0.2) (layer F.Cu) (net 7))
 (segment (start 23.6 22.67) (end 24.3375 22.67) (width 0.2) (layer F.Cu) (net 7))
 (segment (start 22.98 22.67) (end 23.6 22.67) (width 0.2) (layer F.Cu) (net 7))
 (segment (start 19.356 23.644) (end 19.6 23.4) (width 0.2) (layer F.Cu) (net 8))
 (segment (start 19.356 24.46) (end 19.356 23.644) (width 0.2) (layer F.Cu) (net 8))
 (segment (start 23.6 23.17) (end 24.3375 23.17) (width 0.2) (layer F.Cu) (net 8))
 (segment (start 19.6 23.4) (end 22.85 23.4) (width 0.2) (layer F.Cu) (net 8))
 (segment (start 23.08 23.17) (end 23.6 23.17) (width 0.2) (layer F.Cu) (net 8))
 (segment (start 22.85 23.4) (end 23.08 23.17) (width 0.2) (layer F.Cu) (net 8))
 (segment (start 32.67999 22.21999) (end 34.93101 22.21999) (width 0.2) (layer F.Cu) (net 15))
 (segment (start 32.6625 22.17) (end 32.6625 22.2025) (width 0.2) (layer F.Cu) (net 15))
 (segment (start 32.6625 22.2025) (end 32.67999 22.21999) (width 0.2) (layer F.Cu) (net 15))
 (segment (start 35.223 21.928) (end 35.223 20.787) (width 0.2) (layer F.Cu) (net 15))
 (segment (start 34.93101 22.21999) (end 35.223 21.928) (width 0.2) (layer F.Cu) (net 15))
 (segment (start 35.223 18.619) (end 35.222 18.618) (width 0.2) (layer F.Cu) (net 15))
 (segment (start 35.223 20.787) (end 35.223 18.619) (width 0.2) (layer F.Cu) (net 15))
 (segment (start 32.6625 22.67) (end 36.87 22.67) (width 0.2) (layer F.Cu) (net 14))
 (segment (start 37.223 23.023) (end 37.223 24.087) (width 0.2) (layer F.Cu) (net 14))
 (segment (start 36.87 22.67) (end 37.223 23.023) (width 0.2) (layer F.Cu) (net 14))
 (segment (start 37.224 24.088) (end 37.223 24.087) (width 0.2) (layer F.Cu) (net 14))
 (segment (start 39.168 24.088) (end 37.224 24.088) (width 0.2) (layer F.Cu) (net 14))
 (via (at 29.262 24.9172) (size 0.6) (drill 0.3) (layers F.Cu B.Cu) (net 4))
 (segment (start 29.25 24.9292) (end 29.262 24.9172) (width 0.2) (layer F.Cu) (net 4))
 (segment (start 29.25 26.0825) (end 29.25 24.9292) (width 0.2) (layer F.Cu) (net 4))
 (segment (start 27.738 17.094) (end 23.547 17.094) (width 0.2) (layer B.Cu) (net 4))
 (segment (start 29.262 24.9172) (end 28.3476 24.0028) (width 0.2) (layer B.Cu) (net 4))
 (segment (start 28.3476 24.0028) (end 28.3476 17.7036) (width 0.2) (layer B.Cu) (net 4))
 (segment (start 28.3476 17.7036) (end 27.738 17.094) (width 0.2) (layer B.Cu) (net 4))
 (segment (start 23.1025 17.5385) (end 22.0865 17.5385) (width 0.2) (layer B.Cu) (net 4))
 (segment (start 23.547 17.094) (end 23.1025 17.5385) (width 0.2) (layer B.Cu) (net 4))
 (segment (start 22.0865 17.5385) (end 21.388 16.84) (width 0.2) (layer B.Cu) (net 4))
 (segment (start 21.388 16.84) (end 19.408948 16.84) (width 0.2) (layer B.Cu) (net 4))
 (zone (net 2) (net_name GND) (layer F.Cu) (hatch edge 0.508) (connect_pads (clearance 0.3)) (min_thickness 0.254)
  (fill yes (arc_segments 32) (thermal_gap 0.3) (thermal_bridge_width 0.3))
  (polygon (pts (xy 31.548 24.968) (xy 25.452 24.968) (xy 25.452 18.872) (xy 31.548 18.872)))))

